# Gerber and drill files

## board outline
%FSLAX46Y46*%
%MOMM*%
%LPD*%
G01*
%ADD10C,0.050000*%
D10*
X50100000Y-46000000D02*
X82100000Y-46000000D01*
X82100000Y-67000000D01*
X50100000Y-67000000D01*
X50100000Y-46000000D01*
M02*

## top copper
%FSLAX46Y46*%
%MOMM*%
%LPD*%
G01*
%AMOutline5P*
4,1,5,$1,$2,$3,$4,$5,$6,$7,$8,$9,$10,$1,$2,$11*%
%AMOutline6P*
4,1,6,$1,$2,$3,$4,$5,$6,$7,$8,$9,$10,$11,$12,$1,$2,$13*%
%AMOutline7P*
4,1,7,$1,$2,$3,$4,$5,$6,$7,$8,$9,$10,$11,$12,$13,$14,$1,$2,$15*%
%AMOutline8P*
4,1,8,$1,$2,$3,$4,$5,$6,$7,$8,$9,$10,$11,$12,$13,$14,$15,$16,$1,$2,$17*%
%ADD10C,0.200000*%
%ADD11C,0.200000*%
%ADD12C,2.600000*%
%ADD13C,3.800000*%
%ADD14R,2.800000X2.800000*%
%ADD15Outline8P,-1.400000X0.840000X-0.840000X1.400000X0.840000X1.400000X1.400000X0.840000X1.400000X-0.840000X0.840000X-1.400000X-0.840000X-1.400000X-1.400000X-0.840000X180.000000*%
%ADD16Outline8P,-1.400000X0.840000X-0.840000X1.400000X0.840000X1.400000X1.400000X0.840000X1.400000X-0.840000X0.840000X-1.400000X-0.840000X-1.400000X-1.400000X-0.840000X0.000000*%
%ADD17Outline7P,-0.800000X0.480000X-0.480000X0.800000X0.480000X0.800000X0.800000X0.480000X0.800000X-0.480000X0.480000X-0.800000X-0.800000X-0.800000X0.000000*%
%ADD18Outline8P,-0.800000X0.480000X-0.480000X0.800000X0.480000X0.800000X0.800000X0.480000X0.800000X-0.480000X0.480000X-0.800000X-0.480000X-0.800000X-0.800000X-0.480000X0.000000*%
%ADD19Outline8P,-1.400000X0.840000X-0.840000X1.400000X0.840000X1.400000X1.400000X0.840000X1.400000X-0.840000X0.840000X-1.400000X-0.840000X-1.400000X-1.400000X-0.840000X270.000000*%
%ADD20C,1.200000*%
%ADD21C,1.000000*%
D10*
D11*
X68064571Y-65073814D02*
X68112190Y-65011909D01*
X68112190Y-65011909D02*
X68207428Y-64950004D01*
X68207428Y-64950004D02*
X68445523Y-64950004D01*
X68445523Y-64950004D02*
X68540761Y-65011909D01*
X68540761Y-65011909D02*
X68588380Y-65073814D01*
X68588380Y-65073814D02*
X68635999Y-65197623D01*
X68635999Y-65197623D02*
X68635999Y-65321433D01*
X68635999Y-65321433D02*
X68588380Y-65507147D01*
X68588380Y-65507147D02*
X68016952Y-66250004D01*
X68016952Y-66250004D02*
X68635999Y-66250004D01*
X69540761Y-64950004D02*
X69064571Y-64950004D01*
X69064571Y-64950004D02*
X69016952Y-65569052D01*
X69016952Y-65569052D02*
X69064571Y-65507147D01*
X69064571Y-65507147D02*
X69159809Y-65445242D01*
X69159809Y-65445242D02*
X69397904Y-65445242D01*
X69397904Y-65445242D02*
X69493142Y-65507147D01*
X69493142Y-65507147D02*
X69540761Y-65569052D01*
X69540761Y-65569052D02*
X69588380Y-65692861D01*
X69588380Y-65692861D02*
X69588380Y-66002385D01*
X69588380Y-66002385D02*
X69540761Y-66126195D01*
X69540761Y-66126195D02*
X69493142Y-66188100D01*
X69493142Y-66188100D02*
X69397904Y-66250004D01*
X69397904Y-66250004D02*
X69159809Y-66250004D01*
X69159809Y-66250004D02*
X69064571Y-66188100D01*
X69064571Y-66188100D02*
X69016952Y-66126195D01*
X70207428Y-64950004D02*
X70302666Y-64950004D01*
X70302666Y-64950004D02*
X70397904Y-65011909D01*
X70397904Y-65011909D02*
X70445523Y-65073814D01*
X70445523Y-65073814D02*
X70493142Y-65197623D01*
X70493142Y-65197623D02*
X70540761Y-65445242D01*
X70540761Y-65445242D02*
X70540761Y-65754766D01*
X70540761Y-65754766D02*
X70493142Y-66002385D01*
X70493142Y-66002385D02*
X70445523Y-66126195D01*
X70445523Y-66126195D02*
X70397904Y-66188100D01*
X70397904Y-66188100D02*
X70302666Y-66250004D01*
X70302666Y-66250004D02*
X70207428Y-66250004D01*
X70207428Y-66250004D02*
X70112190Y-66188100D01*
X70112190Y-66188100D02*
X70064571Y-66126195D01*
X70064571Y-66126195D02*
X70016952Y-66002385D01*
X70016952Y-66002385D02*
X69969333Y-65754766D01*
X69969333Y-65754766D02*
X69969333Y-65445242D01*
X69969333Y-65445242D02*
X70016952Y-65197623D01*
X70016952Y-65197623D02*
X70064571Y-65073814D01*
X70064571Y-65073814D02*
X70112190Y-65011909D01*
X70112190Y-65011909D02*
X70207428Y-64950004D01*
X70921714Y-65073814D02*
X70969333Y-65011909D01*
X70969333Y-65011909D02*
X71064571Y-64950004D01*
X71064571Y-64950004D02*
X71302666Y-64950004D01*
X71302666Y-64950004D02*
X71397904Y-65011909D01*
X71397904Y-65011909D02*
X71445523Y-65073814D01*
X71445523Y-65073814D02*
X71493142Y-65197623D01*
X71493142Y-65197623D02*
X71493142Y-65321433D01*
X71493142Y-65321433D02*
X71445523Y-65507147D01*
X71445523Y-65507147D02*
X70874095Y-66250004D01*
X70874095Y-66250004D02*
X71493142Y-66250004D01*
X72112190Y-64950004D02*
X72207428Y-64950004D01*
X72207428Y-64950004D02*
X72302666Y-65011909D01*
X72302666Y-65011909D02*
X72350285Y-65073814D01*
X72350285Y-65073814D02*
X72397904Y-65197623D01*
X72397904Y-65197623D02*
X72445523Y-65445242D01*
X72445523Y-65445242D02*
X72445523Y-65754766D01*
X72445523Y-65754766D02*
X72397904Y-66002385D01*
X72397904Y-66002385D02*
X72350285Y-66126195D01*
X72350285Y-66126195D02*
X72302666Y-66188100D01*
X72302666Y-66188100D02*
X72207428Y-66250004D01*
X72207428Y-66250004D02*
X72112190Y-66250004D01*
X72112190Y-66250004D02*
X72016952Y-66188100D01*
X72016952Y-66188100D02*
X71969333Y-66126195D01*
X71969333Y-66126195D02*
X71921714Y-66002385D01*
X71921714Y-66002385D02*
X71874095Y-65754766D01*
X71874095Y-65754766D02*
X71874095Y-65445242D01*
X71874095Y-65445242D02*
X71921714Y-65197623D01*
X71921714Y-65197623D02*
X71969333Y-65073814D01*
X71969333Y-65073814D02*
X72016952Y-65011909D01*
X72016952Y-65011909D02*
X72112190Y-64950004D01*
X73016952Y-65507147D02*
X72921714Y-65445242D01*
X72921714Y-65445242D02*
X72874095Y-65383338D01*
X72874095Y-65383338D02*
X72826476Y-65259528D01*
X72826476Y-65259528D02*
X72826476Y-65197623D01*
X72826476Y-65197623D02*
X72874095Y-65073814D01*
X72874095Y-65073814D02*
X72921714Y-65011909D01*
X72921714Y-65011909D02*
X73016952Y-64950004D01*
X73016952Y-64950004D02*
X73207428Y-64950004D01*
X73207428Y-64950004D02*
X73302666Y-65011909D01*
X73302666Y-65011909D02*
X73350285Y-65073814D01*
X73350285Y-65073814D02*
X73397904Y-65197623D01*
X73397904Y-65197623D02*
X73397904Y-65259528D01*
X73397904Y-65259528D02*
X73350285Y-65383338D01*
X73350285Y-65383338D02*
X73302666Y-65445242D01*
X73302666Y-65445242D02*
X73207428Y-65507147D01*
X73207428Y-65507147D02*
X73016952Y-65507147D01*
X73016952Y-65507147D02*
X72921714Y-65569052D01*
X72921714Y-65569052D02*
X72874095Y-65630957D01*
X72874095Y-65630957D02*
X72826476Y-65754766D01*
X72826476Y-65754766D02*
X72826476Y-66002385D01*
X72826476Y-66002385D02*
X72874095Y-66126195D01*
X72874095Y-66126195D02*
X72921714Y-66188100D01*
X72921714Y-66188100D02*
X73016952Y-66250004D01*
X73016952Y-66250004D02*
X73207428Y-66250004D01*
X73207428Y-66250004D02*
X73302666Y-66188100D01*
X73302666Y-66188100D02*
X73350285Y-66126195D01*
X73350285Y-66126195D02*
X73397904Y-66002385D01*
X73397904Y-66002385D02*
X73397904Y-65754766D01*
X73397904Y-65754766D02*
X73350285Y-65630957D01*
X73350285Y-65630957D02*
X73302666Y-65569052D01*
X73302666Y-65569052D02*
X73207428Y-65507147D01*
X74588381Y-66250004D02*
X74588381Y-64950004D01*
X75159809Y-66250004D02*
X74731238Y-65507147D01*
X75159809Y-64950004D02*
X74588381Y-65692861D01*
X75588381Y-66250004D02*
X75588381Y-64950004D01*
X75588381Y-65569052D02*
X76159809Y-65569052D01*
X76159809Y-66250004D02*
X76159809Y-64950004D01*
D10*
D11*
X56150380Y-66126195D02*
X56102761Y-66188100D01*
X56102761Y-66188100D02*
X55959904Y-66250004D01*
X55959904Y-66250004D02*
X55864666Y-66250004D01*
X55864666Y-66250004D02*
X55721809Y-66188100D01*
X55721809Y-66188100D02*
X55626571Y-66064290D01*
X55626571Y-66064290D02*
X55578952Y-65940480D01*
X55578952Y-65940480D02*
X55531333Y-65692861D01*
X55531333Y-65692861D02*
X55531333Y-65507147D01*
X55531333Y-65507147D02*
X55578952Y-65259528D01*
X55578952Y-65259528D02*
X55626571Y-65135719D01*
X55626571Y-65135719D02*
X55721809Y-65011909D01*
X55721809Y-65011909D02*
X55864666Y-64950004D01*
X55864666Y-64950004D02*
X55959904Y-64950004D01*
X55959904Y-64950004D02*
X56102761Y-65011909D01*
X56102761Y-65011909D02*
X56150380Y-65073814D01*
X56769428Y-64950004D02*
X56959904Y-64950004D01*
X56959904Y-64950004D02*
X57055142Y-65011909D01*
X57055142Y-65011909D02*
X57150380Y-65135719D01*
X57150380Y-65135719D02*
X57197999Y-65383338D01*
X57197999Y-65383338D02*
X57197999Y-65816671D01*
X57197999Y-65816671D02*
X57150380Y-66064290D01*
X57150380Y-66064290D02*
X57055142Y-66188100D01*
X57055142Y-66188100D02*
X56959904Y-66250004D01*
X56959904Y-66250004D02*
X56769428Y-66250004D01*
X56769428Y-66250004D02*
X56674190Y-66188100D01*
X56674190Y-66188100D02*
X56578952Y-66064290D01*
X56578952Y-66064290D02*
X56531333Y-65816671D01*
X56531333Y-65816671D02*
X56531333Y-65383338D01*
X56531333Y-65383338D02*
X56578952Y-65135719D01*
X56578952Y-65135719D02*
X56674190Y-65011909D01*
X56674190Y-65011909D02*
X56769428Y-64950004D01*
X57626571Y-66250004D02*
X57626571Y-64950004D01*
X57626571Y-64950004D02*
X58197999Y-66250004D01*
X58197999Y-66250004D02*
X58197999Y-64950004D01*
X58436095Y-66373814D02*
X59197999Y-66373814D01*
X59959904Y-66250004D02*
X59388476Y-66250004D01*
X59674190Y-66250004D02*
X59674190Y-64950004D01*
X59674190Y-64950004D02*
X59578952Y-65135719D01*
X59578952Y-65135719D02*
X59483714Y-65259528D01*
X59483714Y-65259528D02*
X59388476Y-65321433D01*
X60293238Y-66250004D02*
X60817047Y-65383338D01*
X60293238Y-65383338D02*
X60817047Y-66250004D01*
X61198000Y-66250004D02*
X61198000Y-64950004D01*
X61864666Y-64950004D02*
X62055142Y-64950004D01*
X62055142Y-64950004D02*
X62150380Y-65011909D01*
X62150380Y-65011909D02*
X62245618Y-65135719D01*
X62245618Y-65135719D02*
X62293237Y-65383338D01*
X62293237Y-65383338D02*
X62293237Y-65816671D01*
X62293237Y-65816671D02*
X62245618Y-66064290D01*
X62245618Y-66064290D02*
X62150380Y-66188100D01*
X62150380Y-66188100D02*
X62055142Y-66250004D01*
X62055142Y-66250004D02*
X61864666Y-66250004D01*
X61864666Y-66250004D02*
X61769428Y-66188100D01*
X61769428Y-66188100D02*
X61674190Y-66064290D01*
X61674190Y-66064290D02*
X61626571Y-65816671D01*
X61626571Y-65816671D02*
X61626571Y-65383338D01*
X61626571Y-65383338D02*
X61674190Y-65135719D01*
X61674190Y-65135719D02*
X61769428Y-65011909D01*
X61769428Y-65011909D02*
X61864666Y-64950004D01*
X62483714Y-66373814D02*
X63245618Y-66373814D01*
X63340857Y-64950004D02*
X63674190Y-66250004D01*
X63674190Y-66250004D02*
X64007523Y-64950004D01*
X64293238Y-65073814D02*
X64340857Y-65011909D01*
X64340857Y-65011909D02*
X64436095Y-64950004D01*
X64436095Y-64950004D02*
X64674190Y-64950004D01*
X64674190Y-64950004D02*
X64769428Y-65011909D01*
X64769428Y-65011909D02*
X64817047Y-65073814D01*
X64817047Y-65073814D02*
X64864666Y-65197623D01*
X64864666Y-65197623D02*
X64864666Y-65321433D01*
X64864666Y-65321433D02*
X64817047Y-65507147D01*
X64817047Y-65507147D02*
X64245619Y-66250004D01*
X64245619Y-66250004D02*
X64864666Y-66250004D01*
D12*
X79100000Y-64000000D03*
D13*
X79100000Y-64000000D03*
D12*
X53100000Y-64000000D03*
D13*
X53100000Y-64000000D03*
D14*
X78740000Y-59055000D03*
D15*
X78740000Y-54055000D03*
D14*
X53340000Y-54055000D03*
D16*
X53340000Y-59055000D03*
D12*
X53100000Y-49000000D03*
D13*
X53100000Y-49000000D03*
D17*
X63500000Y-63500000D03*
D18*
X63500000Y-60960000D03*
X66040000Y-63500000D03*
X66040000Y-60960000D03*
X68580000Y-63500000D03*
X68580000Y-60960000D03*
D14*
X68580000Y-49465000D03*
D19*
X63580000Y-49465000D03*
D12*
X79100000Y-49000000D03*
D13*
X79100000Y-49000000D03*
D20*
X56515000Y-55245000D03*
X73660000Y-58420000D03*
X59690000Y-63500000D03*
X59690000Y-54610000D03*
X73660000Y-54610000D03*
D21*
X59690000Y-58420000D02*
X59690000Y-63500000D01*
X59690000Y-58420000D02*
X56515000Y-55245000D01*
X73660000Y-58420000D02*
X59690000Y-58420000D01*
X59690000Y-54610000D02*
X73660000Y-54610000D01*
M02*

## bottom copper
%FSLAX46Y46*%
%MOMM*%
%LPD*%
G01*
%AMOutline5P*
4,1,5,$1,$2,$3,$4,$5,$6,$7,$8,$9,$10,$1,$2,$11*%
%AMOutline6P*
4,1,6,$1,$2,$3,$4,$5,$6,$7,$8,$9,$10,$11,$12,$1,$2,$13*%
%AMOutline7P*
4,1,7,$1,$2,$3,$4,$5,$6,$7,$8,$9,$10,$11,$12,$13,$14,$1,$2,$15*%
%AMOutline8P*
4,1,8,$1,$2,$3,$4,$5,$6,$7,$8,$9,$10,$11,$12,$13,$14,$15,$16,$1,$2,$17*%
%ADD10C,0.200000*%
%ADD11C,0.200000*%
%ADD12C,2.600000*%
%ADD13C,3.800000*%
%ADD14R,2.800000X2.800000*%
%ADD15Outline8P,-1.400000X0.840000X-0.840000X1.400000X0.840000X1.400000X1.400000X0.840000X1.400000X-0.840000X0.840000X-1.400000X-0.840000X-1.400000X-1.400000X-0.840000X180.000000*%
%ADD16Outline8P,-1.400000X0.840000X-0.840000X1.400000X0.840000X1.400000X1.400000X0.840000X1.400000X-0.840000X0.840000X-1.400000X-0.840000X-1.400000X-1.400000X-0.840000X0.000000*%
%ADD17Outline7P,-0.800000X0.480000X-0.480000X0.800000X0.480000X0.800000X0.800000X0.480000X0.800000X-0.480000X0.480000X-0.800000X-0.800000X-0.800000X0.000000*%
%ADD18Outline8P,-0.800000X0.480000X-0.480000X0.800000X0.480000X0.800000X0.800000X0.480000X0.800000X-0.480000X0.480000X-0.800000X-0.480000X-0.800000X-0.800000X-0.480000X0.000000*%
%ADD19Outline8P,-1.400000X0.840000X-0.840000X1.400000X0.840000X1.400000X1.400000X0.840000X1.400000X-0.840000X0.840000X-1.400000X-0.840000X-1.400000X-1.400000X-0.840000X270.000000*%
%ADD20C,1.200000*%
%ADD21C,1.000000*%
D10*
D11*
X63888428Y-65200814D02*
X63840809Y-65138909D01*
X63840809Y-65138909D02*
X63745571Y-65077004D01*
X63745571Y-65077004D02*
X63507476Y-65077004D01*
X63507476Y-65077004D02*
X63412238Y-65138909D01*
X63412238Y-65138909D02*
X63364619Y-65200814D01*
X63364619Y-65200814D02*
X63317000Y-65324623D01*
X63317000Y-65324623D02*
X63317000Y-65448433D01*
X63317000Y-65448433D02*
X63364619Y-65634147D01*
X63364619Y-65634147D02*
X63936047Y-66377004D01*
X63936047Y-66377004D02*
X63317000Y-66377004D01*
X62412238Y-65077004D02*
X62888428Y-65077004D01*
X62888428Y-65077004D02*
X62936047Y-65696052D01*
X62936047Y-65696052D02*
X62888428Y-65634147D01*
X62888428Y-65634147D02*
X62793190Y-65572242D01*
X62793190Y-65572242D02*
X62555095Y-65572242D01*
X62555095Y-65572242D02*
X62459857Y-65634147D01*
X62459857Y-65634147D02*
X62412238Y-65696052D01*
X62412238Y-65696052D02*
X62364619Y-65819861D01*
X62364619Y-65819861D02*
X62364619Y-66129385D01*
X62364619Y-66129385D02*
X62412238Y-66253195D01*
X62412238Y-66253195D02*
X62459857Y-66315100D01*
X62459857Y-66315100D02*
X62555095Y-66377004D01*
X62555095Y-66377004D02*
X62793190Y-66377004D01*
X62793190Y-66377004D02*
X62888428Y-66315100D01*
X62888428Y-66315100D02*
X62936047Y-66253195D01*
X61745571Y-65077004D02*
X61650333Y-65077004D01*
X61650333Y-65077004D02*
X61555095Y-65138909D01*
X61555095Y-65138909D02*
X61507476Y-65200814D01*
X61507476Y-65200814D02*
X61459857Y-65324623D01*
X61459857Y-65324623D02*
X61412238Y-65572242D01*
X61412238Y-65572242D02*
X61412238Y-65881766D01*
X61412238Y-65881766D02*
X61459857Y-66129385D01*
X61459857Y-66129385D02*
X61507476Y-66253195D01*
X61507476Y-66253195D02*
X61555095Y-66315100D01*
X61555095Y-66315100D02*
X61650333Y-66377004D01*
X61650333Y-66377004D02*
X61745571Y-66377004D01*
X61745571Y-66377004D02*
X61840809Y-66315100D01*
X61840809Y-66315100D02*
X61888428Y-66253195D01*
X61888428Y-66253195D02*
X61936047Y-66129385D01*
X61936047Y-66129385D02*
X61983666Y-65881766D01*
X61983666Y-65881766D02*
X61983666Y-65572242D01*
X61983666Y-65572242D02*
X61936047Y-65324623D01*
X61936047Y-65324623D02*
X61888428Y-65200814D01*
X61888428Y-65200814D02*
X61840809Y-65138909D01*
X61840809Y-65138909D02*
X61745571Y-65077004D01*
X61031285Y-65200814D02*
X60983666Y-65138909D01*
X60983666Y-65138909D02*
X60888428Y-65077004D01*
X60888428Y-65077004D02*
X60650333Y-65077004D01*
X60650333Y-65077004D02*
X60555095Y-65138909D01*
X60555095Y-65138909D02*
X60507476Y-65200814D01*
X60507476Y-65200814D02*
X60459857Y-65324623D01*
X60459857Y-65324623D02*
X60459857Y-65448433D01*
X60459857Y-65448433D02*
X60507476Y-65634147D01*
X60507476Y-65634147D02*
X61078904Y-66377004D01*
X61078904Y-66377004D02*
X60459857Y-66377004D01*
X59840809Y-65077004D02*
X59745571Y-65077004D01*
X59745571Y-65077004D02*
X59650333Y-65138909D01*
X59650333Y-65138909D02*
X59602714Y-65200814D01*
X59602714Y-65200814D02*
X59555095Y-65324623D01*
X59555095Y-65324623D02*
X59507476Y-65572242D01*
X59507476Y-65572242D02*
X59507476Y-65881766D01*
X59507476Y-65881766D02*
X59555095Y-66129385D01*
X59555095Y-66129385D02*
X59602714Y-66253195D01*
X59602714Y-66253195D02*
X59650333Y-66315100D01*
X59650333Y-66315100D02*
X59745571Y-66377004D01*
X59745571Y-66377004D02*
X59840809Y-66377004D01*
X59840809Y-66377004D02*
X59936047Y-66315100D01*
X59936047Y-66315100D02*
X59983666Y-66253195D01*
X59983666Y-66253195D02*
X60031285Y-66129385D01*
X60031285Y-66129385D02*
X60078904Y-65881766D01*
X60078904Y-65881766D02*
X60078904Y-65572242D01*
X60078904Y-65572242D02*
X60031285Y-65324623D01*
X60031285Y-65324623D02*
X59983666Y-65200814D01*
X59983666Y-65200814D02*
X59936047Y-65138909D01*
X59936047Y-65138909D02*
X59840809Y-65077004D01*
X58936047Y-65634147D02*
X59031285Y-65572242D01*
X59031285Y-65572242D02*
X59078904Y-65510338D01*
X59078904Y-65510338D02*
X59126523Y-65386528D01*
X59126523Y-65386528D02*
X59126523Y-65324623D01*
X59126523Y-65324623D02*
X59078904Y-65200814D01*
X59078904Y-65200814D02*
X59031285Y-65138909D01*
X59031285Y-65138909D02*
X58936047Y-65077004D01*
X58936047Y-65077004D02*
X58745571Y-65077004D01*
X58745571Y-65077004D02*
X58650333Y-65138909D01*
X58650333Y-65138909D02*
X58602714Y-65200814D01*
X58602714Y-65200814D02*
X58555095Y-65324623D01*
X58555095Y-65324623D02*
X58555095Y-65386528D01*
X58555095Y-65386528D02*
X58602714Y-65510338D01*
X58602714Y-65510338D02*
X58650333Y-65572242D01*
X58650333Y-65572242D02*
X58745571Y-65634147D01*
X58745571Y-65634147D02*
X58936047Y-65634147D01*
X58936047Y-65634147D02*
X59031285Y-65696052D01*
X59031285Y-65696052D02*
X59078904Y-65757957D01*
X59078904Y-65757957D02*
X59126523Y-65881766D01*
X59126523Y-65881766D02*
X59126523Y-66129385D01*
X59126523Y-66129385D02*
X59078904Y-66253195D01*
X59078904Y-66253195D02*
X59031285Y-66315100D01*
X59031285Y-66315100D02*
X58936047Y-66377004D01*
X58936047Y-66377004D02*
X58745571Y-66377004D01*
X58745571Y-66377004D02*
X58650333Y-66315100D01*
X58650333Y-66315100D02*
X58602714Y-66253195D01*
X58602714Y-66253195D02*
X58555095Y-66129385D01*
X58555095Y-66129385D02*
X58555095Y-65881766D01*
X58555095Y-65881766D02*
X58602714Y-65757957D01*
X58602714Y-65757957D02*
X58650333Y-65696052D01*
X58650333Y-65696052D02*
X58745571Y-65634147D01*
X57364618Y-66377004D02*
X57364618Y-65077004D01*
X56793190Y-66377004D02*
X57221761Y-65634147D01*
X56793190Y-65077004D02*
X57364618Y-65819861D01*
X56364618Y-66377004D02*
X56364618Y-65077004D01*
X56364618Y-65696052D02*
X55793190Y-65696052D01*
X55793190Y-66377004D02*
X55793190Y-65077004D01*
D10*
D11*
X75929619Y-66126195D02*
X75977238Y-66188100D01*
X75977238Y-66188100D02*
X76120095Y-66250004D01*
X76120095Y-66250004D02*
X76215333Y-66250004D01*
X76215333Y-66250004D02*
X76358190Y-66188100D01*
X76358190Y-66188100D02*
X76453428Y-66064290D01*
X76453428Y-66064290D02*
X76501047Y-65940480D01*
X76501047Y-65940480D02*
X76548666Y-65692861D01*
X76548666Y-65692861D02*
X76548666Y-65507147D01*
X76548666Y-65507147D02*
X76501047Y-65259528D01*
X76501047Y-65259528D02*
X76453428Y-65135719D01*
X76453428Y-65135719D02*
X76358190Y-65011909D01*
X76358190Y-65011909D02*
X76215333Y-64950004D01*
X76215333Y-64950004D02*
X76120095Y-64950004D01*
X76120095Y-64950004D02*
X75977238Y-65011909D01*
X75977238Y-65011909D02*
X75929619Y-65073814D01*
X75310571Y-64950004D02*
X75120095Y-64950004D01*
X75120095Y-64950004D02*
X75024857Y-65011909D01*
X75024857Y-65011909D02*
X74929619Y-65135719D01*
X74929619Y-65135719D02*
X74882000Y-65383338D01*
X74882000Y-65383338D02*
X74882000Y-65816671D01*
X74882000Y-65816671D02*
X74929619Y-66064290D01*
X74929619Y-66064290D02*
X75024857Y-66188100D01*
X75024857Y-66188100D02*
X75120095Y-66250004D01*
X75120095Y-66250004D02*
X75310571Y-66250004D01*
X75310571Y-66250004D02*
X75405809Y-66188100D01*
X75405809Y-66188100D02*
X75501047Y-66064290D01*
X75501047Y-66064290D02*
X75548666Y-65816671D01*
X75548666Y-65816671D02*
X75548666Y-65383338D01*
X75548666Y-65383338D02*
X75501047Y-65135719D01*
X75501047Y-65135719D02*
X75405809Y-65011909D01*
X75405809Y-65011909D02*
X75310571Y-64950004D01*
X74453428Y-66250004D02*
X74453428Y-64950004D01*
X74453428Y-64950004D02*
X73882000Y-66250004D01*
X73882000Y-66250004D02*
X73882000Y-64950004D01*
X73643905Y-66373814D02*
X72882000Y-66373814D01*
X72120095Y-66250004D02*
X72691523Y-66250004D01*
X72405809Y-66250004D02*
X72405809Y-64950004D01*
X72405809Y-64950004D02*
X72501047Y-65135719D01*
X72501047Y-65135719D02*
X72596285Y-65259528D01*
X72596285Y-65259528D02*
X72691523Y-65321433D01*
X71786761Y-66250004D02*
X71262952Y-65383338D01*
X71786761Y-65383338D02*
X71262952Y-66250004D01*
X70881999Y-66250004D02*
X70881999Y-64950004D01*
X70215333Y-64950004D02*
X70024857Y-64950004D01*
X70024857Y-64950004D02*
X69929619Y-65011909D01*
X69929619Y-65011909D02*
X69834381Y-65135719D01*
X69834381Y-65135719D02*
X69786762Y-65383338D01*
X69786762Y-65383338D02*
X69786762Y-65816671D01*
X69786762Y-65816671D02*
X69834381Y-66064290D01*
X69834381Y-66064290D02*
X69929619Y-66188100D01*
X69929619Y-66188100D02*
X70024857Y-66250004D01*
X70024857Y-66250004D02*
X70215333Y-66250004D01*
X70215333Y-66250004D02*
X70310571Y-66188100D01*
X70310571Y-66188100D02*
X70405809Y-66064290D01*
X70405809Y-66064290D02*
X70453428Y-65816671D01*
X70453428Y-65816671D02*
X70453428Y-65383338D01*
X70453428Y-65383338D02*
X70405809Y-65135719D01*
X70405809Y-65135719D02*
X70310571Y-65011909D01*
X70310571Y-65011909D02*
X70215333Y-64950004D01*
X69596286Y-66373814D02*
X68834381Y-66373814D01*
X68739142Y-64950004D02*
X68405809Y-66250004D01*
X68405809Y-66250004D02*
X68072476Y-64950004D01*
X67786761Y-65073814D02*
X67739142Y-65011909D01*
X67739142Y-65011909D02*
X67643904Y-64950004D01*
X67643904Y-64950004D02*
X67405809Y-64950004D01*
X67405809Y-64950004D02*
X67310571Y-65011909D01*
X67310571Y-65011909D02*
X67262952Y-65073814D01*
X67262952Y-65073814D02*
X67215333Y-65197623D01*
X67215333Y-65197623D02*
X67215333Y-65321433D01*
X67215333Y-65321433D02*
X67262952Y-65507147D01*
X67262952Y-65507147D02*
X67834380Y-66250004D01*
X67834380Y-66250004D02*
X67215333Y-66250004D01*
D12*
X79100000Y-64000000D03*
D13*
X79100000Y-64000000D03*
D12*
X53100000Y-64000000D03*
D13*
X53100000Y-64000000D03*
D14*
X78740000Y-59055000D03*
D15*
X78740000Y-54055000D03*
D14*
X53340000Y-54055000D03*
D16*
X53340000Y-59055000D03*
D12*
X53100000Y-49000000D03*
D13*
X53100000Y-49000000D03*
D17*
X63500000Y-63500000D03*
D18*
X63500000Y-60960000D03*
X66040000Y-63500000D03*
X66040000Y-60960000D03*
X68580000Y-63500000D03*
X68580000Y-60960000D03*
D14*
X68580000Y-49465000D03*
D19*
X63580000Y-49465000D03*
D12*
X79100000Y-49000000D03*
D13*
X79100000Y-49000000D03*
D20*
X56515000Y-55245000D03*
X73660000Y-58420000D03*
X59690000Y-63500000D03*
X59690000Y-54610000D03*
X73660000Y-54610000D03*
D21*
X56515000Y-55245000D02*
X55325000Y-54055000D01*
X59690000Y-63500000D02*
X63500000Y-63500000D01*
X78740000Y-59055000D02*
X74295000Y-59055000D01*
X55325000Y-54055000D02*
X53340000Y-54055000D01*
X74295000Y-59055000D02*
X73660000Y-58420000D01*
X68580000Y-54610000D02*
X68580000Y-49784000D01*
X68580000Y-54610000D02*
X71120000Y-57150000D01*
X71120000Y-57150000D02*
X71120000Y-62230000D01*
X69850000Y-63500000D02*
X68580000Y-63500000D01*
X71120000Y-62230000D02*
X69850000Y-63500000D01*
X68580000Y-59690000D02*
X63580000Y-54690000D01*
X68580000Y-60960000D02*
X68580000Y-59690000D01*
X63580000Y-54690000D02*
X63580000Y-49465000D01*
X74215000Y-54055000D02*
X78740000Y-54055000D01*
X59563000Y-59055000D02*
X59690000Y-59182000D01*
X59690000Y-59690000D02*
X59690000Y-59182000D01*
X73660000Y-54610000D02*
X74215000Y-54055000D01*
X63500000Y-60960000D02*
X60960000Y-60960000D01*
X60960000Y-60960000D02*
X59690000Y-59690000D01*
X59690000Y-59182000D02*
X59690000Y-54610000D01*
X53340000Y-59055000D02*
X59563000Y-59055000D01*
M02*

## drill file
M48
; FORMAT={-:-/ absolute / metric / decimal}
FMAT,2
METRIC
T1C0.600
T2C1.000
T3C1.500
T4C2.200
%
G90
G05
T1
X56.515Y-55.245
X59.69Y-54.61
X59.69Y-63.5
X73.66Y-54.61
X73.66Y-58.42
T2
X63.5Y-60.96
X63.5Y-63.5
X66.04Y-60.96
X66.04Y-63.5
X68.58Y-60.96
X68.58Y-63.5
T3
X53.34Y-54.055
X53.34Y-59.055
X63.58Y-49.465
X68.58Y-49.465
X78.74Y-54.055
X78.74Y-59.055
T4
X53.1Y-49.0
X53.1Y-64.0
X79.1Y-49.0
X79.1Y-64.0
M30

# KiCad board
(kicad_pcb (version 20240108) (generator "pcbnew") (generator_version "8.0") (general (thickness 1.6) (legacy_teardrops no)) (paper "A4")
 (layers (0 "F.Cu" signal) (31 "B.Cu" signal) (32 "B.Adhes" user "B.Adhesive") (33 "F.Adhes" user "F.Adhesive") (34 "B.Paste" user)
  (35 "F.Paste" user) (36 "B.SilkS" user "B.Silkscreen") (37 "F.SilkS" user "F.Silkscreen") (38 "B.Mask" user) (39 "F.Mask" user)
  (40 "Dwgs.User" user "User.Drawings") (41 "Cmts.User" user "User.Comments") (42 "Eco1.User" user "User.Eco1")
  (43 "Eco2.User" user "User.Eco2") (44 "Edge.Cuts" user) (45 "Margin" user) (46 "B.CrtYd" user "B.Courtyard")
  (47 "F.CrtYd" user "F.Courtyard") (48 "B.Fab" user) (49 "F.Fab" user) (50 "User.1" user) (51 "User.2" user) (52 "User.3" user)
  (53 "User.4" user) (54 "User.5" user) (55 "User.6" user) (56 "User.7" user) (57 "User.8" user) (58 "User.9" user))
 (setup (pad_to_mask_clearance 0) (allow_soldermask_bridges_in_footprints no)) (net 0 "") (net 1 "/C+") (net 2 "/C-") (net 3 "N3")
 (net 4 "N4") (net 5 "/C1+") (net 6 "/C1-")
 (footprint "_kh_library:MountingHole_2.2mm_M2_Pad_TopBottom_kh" (layer "F.Cu") (at 79.1 64)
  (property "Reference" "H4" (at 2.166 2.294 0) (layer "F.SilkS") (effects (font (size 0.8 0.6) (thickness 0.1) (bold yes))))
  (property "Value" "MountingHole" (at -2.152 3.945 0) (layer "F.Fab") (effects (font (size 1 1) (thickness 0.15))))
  (pad "1" thru_hole circle (at 0 0) (size 2.6 2.6) (drill 2.2) (layers "*.Cu" "*.Mask") (remove_unused_layers no))
  (pad "1" connect circle (at 0 0) (size 3.8 3.8) (layers "F.Cu" "F.Mask"))
  (pad "1" connect circle (at 0 0) (size 3.8 3.8) (layers "B.Cu" "B.Mask")))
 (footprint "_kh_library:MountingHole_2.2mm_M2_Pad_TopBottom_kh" (layer "F.Cu") (at 53.1 64)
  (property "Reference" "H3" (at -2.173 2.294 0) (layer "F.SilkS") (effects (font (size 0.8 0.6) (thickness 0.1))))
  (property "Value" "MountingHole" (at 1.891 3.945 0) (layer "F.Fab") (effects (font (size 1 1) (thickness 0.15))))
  (pad "1" thru_hole circle (at 0 0) (size 2.6 2.6) (drill 2.2) (layers "*.Cu" "*.Mask") (remove_unused_layers no))
  (pad "1" connect circle (at 0 0) (size 3.8 3.8) (layers "F.Cu" "F.Mask"))
  (pad "1" connect circle (at 0 0) (size 3.8 3.8) (layers "B.Cu" "B.Mask")))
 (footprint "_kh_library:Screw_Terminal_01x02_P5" (layer "F.Cu") (at 78.74 59.055 180)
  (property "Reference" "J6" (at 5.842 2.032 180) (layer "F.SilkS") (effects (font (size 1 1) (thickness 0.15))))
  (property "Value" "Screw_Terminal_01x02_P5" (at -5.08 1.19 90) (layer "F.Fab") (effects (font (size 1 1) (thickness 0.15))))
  (pad "1" thru_hole rect (at 0 0 180) (size 2.8 2.8) (drill 1.5) (layers "*.Cu" "*.Mask") (remove_unused_layers no) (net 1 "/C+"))
  (pad "2" thru_hole roundrect (at 0 5 180) (size 2.8 2.8) (drill 1.5) (layers "*.Cu" "*.Mask") (remove_unused_layers no)
   (roundrect_rratio 0) (chamfer_ratio 0.2) (chamfer top_left top_right bottom_left bottom_right) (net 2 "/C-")))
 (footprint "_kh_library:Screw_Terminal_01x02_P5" (layer "F.Cu") (at 53.34 54.055)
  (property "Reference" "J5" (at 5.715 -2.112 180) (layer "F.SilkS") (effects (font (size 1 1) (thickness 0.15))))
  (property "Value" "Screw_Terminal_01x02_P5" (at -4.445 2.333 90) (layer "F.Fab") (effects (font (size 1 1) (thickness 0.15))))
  (pad "1" thru_hole rect (at 0 0) (size 2.8 2.8) (drill 1.5) (layers "*.Cu" "*.Mask") (remove_unused_layers no) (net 1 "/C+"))
  (pad "2" thru_hole roundrect (at 0 5) (size 2.8 2.8) (drill 1.5) (layers "*.Cu" "*.Mask") (remove_unused_layers no) (roundrect_rratio 0)
   (chamfer_ratio 0.2) (chamfer top_left top_right bottom_left bottom_right) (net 2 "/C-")))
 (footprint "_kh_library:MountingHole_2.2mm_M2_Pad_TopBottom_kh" (layer "F.Cu") (at 53.1 49)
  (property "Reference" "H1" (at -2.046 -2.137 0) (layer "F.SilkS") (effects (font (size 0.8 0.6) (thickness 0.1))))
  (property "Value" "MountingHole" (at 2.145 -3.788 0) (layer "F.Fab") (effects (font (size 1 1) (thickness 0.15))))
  (pad "1" thru_hole circle (at 0 0) (size 2.6 2.6) (drill 2.2) (layers "*.Cu" "*.Mask") (remove_unused_layers no))
  (pad "1" connect circle (at 0 0) (size 3.8 3.8) (layers "F.Cu" "F.Mask"))
  (pad "1" connect circle (at 0 0) (size 3.8 3.8) (layers "B.Cu" "B.Mask")))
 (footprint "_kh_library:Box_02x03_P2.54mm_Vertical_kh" (layer "F.Cu") (at 63.5 63.5)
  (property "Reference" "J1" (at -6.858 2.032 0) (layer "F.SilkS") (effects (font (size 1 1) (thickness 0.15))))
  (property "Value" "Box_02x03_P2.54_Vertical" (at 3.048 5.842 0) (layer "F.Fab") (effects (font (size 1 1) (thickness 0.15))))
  (pad "1" thru_hole roundrect (at 0 0) (size 1.6 1.6) (drill 1) (layers "*.Cu" "*.Mask") (remove_unused_layers no) (roundrect_rratio 0)
   (chamfer_ratio 0.2) (chamfer top_left top_right bottom_right) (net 1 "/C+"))
  (pad "2" thru_hole roundrect (at 0 -2.54) (size 1.6 1.6) (drill 1) (layers "*.Cu" "*.Mask") (remove_unused_layers no) (roundrect_rratio 0)
   (chamfer_ratio 0.2) (chamfer top_left top_right bottom_left bottom_right) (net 2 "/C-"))
  (pad "3" thru_hole roundrect (at 2.54 0) (size 1.6 1.6) (drill 1) (layers "*.Cu" "*.Mask") (remove_unused_layers no) (roundrect_rratio 0)
   (chamfer_ratio 0.2) (chamfer top_left top_right bottom_left bottom_right) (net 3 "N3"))
  (pad "4" thru_hole roundrect (at 2.54 -2.54) (size 1.6 1.6) (drill 1) (layers "*.Cu" "*.Mask") (remove_unused_layers no)
   (roundrect_rratio 0) (chamfer_ratio 0.2) (chamfer top_left top_right bottom_left bottom_right) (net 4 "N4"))
  (pad "5" thru_hole roundrect (at 5.08 0) (size 1.6 1.6) (drill 1) (layers "*.Cu" "*.Mask") (remove_unused_layers no) (roundrect_rratio 0)
   (chamfer_ratio 0.2) (chamfer top_left top_right bottom_left bottom_right) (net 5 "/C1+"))
  (pad "6" thru_hole roundrect (at 5.08 -2.54) (size 1.6 1.6) (drill 1) (layers "*.Cu" "*.Mask") (remove_unused_layers no)
   (roundrect_rratio 0) (chamfer_ratio 0.2) (chamfer top_left top_right bottom_left bottom_right) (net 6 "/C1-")))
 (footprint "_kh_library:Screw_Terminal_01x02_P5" (layer "F.Cu") (at 68.58 49.465 -90)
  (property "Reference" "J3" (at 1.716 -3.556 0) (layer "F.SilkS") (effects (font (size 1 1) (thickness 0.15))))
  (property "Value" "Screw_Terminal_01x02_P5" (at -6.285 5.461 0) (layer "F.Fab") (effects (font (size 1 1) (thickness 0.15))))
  (pad "1" thru_hole rect (at 0 0 270) (size 2.8 2.8) (drill 1.5) (layers "*.Cu" "*.Mask") (remove_unused_layers no) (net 5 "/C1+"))
  (pad "2" thru_hole roundrect (at 0 5 270) (size 2.8 2.8) (drill 1.5) (layers "*.Cu" "*.Mask") (remove_unused_layers no)
   (roundrect_rratio 0) (chamfer_ratio 0.2) (chamfer top_left top_right bottom_left bottom_right) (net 6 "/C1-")))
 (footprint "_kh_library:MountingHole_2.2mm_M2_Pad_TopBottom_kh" (layer "F.Cu") (at 79.1 49)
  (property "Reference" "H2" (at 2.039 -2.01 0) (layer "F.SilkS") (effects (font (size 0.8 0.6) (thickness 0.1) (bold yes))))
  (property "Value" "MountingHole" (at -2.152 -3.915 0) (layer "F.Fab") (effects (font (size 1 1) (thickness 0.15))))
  (pad "1" thru_hole circle (at 0 0) (size 2.6 2.6) (drill 2.2) (layers "*.Cu" "*.Mask") (remove_unused_layers no))
  (pad "1" connect circle (at 0 0) (size 3.8 3.8) (layers "F.Cu" "F.Mask"))
  (pad "1" connect circle (at 0 0) (size 3.8 3.8) (layers "B.Cu" "B.Mask")))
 (gr_rect (start 50.1 46) (end 82.1 67) (stroke (width 0.05) (type default)) (fill none) (layer "Edge.Cuts"))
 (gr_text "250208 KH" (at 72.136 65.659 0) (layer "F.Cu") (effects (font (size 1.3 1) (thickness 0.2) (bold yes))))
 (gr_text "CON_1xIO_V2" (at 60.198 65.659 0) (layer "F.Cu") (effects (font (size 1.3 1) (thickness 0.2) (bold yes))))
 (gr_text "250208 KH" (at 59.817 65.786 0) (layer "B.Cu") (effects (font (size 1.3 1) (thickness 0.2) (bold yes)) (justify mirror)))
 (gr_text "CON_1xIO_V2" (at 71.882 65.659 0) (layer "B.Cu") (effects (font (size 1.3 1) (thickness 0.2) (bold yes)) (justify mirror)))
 (segment (start 59.69 58.42) (end 59.69 63.5) (width 1) (layer "F.Cu") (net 1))
 (segment (start 59.69 58.42) (end 56.515 55.245) (width 1) (layer "F.Cu") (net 1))
 (segment (start 73.66 58.42) (end 59.69 58.42) (width 1) (layer "F.Cu") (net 1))
 (via (at 56.515 55.245) (size 1.2) (drill 0.6) (layers "F.Cu" "B.Cu") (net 1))
 (via (at 73.66 58.42) (size 1.2) (drill 0.6) (layers "F.Cu" "B.Cu") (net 1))
 (via (at 59.69 63.5) (size 1.2) (drill 0.6) (layers "F.Cu" "B.Cu") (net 1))
 (segment (start 56.515 55.245) (end 55.325 54.055) (width 1) (layer "B.Cu") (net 1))
 (segment (start 59.69 63.5) (end 63.5 63.5) (width 1) (layer "B.Cu") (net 1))
 (segment (start 78.74 59.055) (end 74.295 59.055) (width 1) (layer "B.Cu") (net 1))
 (segment (start 55.325 54.055) (end 53.34 54.055) (width 1) (layer "B.Cu") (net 1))
 (segment (start 74.295 59.055) (end 73.66 58.42) (width 1) (layer "B.Cu") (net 1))
 (segment (start 68.58 54.61) (end 68.58 49.784) (width 1) (layer "B.Cu") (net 5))
 (segment (start 68.58 54.61) (end 71.12 57.15) (width 1) (layer "B.Cu") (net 5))
 (segment (start 71.12 57.15) (end 71.12 62.23) (width 1) (layer "B.Cu") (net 5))
 (segment (start 69.85 63.5) (end 68.58 63.5) (width 1) (layer "B.Cu") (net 5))
 (segment (start 71.12 62.23) (end 69.85 63.5) (width 1) (layer "B.Cu") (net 5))
 (segment (start 68.58 59.69) (end 63.58 54.69) (width 1) (layer "B.Cu") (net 6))
 (segment (start 68.58 60.96) (end 68.58 59.69) (width 1) (layer "B.Cu") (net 6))
 (segment (start 63.58 54.69) (end 63.58 49.465) (width 1) (layer "B.Cu") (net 6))
 (segment (start 59.69 54.61) (end 73.66 54.61) (width 1) (layer "F.Cu") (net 2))
 (via (at 59.69 54.61) (size 1.2) (drill 0.6) (layers "F.Cu" "B.Cu") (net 2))
 (via (at 73.66 54.61) (size 1.2) (drill 0.6) (layers "F.Cu" "B.Cu") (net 2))
 (segment (start 74.215 54.055) (end 78.74 54.055) (width 1) (layer "B.Cu") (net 2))
 (segment (start 59.563 59.055) (end 59.69 59.182) (width 1) (layer "B.Cu") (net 2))
 (segment (start 59.69 59.69) (end 59.69 59.182) (width 1) (layer "B.Cu") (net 2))
 (segment (start 73.66 54.61) (end 74.215 54.055) (width 1) (layer "B.Cu") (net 2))
 (segment (start 63.5 60.96) (end 60.96 60.96) (width 1) (layer "B.Cu") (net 2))
 (segment (start 60.96 60.96) (end 59.69 59.69) (width 1) (layer "B.Cu") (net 2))
 (segment (start 59.69 59.182) (end 59.69 54.61) (width 1) (layer "B.Cu") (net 2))
 (segment (start 53.34 59.055) (end 59.563 59.055) (width 1) (layer "B.Cu") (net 2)))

